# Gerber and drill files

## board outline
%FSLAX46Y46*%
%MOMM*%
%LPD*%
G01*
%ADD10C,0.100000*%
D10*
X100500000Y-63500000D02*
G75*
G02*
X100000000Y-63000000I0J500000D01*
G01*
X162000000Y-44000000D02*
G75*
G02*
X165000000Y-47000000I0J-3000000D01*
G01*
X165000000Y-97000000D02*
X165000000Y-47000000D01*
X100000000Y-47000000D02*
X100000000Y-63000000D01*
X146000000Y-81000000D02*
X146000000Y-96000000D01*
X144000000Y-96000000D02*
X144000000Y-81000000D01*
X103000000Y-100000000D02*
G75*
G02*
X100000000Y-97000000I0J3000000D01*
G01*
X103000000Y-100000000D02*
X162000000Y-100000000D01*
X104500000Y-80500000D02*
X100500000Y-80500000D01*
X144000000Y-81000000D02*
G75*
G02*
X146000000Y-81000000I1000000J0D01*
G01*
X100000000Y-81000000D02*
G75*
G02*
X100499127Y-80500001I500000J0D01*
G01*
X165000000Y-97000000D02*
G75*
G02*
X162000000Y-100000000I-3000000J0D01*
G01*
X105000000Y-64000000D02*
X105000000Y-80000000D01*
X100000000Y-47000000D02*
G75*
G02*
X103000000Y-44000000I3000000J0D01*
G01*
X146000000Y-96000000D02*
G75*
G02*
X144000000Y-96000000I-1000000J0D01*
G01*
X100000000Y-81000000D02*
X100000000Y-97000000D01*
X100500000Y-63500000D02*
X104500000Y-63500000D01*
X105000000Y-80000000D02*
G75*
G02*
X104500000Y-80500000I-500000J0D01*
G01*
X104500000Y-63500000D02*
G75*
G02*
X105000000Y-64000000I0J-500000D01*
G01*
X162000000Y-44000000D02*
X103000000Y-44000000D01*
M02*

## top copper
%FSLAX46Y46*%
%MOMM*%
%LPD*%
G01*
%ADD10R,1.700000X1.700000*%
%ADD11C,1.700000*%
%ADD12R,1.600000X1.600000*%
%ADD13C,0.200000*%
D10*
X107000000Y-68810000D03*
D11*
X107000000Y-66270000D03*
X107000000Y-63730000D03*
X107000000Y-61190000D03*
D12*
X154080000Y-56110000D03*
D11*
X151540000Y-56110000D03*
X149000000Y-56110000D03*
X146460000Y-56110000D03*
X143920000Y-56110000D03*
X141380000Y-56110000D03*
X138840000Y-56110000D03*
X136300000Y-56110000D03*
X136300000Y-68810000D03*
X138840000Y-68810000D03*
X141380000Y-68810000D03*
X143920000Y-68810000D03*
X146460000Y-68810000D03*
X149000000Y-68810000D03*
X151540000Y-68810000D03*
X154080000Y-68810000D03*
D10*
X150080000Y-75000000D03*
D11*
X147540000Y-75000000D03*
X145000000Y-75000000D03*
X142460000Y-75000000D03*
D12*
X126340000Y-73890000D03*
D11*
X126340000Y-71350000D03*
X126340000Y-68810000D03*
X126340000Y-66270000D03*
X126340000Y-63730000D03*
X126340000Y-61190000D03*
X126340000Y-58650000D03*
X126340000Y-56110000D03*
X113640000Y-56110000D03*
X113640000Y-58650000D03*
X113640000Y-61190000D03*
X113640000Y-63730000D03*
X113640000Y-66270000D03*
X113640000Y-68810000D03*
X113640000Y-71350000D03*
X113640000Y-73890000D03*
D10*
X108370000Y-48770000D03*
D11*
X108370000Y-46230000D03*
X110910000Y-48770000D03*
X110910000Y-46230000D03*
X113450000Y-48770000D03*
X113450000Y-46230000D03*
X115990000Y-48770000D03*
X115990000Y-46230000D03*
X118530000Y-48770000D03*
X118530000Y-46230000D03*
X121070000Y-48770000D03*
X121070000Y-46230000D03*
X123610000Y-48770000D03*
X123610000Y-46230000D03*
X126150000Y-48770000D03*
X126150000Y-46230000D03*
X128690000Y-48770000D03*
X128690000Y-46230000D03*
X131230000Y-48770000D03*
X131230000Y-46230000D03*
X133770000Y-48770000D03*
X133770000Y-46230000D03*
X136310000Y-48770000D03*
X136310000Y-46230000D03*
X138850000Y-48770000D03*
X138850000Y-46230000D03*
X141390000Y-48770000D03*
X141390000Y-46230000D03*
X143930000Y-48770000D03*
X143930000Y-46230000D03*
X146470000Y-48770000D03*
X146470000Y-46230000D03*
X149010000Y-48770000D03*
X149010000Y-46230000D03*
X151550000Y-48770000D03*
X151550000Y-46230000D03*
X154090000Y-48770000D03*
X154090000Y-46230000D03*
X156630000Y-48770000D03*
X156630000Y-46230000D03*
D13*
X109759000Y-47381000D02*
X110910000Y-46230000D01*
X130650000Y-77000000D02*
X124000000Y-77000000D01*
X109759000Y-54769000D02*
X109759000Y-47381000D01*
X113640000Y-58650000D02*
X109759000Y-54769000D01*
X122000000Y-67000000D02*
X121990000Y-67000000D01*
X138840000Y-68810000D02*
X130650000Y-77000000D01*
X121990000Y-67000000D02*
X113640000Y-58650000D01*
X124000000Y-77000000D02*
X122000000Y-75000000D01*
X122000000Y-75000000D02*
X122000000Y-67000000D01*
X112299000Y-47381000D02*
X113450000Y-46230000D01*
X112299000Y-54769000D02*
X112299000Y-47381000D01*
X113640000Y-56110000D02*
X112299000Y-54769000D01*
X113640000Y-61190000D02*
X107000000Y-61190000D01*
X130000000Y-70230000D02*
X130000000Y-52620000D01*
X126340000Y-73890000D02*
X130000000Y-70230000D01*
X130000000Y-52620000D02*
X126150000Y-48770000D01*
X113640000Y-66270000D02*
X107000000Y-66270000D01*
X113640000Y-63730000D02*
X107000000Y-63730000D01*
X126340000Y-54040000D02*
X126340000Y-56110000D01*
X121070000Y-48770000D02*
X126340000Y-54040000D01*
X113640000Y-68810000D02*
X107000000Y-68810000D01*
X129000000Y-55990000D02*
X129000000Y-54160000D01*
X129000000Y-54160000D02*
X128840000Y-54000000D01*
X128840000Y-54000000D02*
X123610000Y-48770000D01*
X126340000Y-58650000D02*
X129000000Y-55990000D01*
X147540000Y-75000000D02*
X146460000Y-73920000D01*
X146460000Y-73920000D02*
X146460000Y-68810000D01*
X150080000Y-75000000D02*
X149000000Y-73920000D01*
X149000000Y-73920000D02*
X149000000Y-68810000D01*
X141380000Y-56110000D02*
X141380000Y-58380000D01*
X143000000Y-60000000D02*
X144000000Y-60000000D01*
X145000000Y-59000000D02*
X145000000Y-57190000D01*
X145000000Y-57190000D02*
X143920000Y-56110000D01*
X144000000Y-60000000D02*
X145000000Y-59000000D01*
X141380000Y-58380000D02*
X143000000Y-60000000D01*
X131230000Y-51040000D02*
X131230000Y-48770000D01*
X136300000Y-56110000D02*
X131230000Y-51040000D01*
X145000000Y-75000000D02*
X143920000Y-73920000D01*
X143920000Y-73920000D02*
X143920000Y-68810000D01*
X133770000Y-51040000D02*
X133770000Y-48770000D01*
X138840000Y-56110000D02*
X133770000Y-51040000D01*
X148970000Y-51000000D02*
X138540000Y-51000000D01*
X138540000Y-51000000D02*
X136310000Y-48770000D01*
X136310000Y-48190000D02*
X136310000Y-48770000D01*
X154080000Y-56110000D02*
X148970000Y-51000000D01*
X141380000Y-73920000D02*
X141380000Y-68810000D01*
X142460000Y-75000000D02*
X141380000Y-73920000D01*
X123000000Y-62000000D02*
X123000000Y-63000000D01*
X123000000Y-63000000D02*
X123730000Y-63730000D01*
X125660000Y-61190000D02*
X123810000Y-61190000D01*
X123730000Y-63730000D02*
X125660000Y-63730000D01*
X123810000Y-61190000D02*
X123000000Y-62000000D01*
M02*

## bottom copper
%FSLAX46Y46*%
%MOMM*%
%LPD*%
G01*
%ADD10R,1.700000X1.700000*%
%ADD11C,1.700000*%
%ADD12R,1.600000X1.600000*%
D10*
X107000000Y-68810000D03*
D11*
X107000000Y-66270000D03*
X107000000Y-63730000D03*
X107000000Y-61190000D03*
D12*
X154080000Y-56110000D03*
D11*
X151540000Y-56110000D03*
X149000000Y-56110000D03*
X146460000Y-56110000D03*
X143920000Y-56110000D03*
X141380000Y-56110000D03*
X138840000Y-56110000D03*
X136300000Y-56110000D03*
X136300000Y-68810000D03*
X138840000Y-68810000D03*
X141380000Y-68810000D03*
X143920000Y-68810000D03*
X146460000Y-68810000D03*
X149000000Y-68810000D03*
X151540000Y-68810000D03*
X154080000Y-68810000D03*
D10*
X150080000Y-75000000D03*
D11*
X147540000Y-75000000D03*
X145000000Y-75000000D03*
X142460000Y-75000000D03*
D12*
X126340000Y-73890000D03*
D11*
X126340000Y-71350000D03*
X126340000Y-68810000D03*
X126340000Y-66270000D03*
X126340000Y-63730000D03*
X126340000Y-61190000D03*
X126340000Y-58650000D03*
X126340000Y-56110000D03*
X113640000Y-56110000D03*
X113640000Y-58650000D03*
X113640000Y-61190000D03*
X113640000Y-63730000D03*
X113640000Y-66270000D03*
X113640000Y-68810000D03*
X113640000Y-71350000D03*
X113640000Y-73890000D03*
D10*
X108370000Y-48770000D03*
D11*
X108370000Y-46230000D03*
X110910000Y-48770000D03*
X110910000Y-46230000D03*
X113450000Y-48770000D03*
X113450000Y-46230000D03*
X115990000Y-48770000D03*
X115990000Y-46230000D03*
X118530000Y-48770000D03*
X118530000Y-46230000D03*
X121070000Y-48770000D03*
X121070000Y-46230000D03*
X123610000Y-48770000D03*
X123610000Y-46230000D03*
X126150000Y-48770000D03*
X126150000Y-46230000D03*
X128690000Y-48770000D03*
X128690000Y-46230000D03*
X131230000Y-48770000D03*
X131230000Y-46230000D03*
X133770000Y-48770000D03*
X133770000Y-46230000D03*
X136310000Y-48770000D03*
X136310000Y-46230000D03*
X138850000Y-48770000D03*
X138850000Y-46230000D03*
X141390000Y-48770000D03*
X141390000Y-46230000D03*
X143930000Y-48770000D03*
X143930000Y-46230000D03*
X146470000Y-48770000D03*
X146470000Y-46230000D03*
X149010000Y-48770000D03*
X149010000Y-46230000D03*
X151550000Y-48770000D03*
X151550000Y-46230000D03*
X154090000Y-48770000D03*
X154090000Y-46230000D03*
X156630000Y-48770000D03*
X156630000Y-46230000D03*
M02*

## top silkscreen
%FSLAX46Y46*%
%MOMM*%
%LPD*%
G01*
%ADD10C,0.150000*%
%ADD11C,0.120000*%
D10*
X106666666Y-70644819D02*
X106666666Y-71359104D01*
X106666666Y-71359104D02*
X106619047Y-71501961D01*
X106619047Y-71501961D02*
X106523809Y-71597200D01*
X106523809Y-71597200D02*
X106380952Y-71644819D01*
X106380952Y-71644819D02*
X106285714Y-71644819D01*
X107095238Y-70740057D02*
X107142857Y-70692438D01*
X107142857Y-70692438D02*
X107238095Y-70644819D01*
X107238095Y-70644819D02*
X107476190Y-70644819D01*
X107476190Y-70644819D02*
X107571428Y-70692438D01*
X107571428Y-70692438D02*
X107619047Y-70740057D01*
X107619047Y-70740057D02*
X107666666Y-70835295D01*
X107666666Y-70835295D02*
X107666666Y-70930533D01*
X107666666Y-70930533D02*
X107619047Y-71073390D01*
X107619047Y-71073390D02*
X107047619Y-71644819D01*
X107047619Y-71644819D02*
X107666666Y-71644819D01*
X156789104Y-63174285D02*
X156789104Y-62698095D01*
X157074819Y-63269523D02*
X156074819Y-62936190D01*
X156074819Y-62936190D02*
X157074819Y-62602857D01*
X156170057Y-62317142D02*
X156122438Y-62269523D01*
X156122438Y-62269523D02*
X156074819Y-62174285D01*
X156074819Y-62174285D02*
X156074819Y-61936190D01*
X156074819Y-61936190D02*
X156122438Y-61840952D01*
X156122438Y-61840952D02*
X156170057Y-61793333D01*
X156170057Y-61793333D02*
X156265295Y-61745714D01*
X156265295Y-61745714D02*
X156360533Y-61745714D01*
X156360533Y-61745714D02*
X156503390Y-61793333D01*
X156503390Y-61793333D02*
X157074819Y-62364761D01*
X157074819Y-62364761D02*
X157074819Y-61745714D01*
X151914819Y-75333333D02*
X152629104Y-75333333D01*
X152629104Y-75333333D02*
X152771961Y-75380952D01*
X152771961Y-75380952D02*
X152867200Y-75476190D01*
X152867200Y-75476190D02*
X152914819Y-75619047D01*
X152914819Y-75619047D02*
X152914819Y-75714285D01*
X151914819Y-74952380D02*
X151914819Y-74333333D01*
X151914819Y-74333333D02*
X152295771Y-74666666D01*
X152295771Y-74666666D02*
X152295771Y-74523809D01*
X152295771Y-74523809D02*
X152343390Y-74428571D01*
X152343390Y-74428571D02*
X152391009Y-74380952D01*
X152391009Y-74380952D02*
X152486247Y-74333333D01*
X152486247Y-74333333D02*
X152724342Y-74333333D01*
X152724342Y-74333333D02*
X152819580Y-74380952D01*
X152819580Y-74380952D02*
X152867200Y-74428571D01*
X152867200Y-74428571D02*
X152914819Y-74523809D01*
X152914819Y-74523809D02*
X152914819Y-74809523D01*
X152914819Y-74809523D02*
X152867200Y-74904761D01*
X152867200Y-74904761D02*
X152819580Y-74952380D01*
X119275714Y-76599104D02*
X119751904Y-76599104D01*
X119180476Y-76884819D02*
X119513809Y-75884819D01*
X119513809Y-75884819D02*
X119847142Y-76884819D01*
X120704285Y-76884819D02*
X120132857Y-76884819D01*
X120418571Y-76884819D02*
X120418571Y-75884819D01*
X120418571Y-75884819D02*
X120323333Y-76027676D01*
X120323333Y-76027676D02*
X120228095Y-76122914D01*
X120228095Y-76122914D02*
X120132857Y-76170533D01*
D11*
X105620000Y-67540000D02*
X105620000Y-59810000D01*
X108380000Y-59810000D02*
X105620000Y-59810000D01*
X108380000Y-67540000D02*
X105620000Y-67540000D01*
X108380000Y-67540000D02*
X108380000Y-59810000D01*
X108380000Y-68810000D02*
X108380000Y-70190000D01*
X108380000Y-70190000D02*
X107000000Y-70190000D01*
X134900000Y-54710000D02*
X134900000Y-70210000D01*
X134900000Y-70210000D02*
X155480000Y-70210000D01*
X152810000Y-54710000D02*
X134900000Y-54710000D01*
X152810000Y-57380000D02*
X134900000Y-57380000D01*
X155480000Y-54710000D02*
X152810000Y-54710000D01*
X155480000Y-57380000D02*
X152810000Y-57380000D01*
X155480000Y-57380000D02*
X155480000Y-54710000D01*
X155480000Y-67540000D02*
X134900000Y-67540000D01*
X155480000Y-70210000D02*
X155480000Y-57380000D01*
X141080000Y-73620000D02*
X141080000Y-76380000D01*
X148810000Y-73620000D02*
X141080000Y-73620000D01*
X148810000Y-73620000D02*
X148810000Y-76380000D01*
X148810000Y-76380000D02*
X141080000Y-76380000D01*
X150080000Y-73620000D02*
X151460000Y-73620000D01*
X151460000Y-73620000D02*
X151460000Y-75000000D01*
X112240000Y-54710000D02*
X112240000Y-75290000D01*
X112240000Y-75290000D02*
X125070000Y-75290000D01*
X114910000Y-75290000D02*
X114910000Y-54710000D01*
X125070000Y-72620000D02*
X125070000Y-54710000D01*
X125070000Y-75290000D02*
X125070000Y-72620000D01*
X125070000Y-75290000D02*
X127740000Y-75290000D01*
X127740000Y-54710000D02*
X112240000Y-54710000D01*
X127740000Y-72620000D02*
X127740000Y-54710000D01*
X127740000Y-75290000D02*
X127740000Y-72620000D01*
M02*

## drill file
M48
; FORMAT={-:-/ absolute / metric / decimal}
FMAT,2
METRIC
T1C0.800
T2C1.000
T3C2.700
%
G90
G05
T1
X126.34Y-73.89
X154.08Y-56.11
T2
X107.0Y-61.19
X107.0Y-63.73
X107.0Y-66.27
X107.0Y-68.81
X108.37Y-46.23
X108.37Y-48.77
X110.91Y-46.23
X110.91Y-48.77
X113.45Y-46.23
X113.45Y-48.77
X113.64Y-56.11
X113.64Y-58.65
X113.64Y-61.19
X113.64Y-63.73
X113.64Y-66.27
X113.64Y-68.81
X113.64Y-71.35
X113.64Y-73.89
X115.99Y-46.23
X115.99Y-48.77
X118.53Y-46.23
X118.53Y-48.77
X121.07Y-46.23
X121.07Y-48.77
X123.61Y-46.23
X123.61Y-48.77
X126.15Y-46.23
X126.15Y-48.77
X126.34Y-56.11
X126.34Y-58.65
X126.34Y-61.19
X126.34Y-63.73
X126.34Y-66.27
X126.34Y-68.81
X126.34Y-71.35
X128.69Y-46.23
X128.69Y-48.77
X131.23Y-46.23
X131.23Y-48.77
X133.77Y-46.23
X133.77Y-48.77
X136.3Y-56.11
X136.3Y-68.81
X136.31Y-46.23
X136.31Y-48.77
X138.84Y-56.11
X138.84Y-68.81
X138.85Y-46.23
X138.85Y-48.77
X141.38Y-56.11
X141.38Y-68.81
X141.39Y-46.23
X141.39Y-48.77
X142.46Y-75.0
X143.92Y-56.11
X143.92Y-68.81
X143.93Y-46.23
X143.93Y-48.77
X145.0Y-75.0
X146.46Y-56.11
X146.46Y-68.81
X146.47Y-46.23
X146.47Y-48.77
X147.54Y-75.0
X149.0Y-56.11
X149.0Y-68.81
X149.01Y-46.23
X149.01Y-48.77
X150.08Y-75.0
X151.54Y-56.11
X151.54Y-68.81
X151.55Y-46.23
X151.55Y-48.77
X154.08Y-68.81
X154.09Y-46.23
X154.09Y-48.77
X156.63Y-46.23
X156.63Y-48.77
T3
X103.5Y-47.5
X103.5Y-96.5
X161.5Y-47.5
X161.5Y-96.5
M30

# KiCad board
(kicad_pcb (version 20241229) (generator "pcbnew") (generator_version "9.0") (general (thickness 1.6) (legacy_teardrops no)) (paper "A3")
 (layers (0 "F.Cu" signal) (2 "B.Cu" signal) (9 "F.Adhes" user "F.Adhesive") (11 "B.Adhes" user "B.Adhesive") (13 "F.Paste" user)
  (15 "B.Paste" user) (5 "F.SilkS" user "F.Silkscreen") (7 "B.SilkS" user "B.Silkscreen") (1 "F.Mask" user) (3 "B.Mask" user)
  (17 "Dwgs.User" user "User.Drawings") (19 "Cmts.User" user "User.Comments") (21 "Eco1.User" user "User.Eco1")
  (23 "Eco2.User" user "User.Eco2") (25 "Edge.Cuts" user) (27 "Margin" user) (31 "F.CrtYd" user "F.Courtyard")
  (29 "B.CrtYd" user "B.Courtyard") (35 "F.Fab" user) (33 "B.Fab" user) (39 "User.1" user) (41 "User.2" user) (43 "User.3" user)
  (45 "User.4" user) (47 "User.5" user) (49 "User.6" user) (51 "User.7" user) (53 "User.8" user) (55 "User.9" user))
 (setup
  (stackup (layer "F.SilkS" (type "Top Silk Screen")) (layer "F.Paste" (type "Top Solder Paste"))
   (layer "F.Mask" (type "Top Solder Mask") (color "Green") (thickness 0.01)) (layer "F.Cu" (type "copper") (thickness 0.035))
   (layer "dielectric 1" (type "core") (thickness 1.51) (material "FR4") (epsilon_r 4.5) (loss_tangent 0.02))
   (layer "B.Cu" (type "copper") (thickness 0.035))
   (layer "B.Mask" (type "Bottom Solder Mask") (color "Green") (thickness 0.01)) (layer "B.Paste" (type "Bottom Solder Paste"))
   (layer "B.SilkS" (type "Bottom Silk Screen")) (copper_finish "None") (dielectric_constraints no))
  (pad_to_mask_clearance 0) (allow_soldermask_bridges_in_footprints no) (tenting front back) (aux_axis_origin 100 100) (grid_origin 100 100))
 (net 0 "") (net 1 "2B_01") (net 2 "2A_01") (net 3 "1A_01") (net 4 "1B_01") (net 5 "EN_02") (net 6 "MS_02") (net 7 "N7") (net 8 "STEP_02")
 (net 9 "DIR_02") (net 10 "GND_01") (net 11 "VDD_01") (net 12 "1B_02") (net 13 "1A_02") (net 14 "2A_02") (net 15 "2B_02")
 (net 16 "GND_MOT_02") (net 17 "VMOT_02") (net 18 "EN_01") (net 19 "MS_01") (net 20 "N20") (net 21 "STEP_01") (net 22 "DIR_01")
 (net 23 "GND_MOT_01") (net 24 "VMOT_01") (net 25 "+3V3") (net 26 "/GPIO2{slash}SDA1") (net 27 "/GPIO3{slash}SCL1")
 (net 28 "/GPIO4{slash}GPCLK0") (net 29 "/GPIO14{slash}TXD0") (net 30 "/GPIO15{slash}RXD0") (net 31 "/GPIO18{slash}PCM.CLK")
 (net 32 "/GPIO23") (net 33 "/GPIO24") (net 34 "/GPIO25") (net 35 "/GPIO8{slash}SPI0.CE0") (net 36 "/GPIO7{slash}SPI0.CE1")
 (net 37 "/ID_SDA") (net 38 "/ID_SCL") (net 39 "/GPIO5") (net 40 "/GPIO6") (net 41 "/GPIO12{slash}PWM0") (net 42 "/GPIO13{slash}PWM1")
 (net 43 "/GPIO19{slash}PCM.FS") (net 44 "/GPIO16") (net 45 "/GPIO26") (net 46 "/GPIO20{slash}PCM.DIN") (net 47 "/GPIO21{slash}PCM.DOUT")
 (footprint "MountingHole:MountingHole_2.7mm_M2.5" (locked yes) (layer "F.Cu") (at 161.5 47.5)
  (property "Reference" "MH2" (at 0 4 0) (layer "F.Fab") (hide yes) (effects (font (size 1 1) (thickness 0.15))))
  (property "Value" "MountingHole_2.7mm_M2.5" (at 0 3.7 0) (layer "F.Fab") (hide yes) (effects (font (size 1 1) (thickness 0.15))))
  (pad "" np_thru_hole circle (at 0 0) (size 2.7 2.7) (drill 2.7) (layers "*.Cu" "*.Mask")))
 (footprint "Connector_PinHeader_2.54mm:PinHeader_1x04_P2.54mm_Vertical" (layer "F.Cu") (at 107 68.81 180)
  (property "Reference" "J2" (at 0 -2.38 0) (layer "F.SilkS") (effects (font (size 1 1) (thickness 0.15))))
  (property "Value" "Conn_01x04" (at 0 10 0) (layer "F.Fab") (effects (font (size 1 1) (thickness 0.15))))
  (fp_line (start 1.38 1.27) (end 1.38 9) (stroke (width 0.12) (type solid)) (layer "F.SilkS"))
  (fp_line (start -1.38 9) (end 1.38 9) (stroke (width 0.12) (type solid)) (layer "F.SilkS"))
  (fp_line (start -1.38 1.27) (end 1.38 1.27) (stroke (width 0.12) (type solid)) (layer "F.SilkS"))
  (fp_line (start -1.38 1.27) (end -1.38 9) (stroke (width 0.12) (type solid)) (layer "F.SilkS"))
  (fp_line (start -1.38 0) (end -1.38 -1.38) (stroke (width 0.12) (type solid)) (layer "F.SilkS"))
  (fp_line (start -1.38 -1.38) (end 0 -1.38) (stroke (width 0.12) (type solid)) (layer "F.SilkS"))
  (pad "1" thru_hole rect (at 0 0 180) (size 1.7 1.7) (drill 1) (layers "*.Cu" "*.Mask") (remove_unused_layers no) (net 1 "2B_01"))
  (pad "2" thru_hole circle (at 0 2.54 180) (size 1.7 1.7) (drill 1) (layers "*.Cu" "*.Mask") (remove_unused_layers no) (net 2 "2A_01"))
  (pad "3" thru_hole circle (at 0 5.08 180) (size 1.7 1.7) (drill 1) (layers "*.Cu" "*.Mask") (remove_unused_layers no) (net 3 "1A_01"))
  (pad "4" thru_hole circle (at 0 7.62 180) (size 1.7 1.7) (drill 1) (layers "*.Cu" "*.Mask") (remove_unused_layers no) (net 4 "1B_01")))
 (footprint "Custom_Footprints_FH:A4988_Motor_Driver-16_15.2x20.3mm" (layer "F.Cu") (at 154.08 56.11 -90)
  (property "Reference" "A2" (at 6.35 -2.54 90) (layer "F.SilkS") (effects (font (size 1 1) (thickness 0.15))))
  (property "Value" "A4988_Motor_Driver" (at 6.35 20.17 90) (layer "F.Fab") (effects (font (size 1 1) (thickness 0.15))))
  (fp_line (start -1.4 19.18) (end 14.1 19.18) (stroke (width 0.12) (type solid)) (layer "F.SilkS"))
  (fp_line (start 14.1 19.18) (end 14.1 -1.4) (stroke (width 0.12) (type solid)) (layer "F.SilkS"))
  (fp_line (start -1.4 1.27) (end -1.4 19.18) (stroke (width 0.12) (type solid)) (layer "F.SilkS"))
  (fp_line (start 1.27 1.27) (end 1.27 19.18) (stroke (width 0.12) (type solid)) (layer "F.SilkS"))
  (fp_line (start -1.4 -1.4) (end -1.4 1.27) (stroke (width 0.12) (type solid)) (layer "F.SilkS"))
  (fp_line (start 1.27 -1.4) (end 1.27 1.27) (stroke (width 0.12) (type solid)) (layer "F.SilkS"))
  (fp_line (start 1.27 -1.4) (end -1.4 -1.4) (stroke (width 0.12) (type solid)) (layer "F.SilkS"))
  (fp_line (start 11.43 -1.4) (end 11.43 19.18) (stroke (width 0.12) (type solid)) (layer "F.SilkS"))
  (fp_line (start 14.1 -1.4) (end 1.27 -1.4) (stroke (width 0.12) (type solid)) (layer "F.SilkS"))
  (pad "1" thru_hole rect (at 0 0 270) (size 1.6 1.6) (drill 0.8) (layers "*.Cu" "*.Mask") (remove_unused_layers no) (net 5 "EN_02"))
  (pad "2" thru_hole circle (at 0 2.54 270) (size 1.7 1.7) (drill 1) (layers "*.Cu" "*.Mask") (remove_unused_layers no) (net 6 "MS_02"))
  (pad "3" thru_hole circle (at 0 5.08 270) (size 1.7 1.7) (drill 1) (layers "*.Cu" "*.Mask") (remove_unused_layers no) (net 6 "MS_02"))
  (pad "4" thru_hole circle (at 0 7.62 270) (size 1.7 1.7) (drill 1) (layers "*.Cu" "*.Mask") (remove_unused_layers no) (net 6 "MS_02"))
  (pad "5" thru_hole circle (at 0 10.16 270) (size 1.7 1.7) (drill 1) (layers "*.Cu" "*.Mask") (remove_unused_layers no) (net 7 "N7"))
  (pad "6" thru_hole circle (at 0 12.7 270) (size 1.7 1.7) (drill 1) (layers "*.Cu" "*.Mask") (remove_unused_layers no) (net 7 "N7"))
  (pad "7" thru_hole circle (at 0 15.24 270) (size 1.7 1.7) (drill 1) (layers "*.Cu" "*.Mask") (remove_unused_layers no) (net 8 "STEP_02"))
  (pad "8" thru_hole circle (at 0 17.78 270) (size 1.7 1.7) (drill 1) (layers "*.Cu" "*.Mask") (remove_unused_layers no) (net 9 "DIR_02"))
  (pad "9" thru_hole circle (at 12.7 17.78 270) (size 1.7 1.7) (drill 1) (layers "*.Cu" "*.Mask") (remove_unused_layers no)
   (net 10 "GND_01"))
  (pad "10" thru_hole circle (at 12.7 15.24 270) (size 1.7 1.7) (drill 1) (layers "*.Cu" "*.Mask") (remove_unused_layers no)
   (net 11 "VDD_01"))
  (pad "11" thru_hole circle (at 12.7 12.7 270) (size 1.7 1.7) (drill 1) (layers "*.Cu" "*.Mask") (remove_unused_layers no) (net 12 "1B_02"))
  (pad "12" thru_hole circle (at 12.7 10.16 270) (size 1.7 1.7) (drill 1) (layers "*.Cu" "*.Mask") (remove_unused_layers no)
   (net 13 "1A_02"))
  (pad "13" thru_hole circle (at 12.7 7.62 270) (size 1.7 1.7) (drill 1) (layers "*.Cu" "*.Mask") (remove_unused_layers no) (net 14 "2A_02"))
  (pad "14" thru_hole circle (at 12.7 5.08 270) (size 1.7 1.7) (drill 1) (layers "*.Cu" "*.Mask") (remove_unused_layers no) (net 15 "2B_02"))
  (pad "15" thru_hole circle (at 12.7 2.54 270) (size 1.7 1.7) (drill 1) (layers "*.Cu" "*.Mask") (remove_unused_layers no)
   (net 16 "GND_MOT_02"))
  (pad "16" thru_hole circle (at 12.7 0 270) (size 1.7 1.7) (drill 1) (layers "*.Cu" "*.Mask") (remove_unused_layers no) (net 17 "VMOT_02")))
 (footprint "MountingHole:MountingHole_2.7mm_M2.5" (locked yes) (layer "F.Cu") (at 103.5 96.5)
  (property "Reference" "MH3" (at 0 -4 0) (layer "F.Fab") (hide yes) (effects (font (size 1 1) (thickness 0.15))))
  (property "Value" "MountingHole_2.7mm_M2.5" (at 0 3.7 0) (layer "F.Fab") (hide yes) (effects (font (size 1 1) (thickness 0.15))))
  (pad "" np_thru_hole circle (at 0 0) (size 2.7 2.7) (drill 2.7) (layers "*.Cu" "*.Mask")))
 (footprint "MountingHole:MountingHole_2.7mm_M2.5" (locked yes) (layer "F.Cu") (at 103.5 47.5)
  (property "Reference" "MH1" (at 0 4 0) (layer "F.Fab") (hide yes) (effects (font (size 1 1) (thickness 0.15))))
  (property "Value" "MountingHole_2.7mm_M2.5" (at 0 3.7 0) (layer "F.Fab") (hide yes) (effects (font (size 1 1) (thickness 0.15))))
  (pad "" np_thru_hole circle (at 0 0) (size 2.7 2.7) (drill 2.7) (layers "*.Cu" "*.Mask")))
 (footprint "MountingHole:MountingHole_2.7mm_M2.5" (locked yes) (layer "F.Cu") (at 161.5 96.5)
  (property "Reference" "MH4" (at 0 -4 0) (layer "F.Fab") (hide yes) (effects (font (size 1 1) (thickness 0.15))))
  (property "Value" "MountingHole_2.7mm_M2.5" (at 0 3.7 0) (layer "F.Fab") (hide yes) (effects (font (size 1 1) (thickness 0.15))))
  (pad "" np_thru_hole circle (at 0 0) (size 2.7 2.7) (drill 2.7) (layers "*.Cu" "*.Mask")))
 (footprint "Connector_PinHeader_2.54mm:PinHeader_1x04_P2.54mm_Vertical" (layer "F.Cu") (at 150.08 75 -90)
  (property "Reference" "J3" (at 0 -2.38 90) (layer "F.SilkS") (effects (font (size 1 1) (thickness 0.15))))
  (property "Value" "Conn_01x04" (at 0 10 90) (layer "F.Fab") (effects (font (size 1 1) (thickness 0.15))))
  (fp_line (start -1.38 9) (end 1.38 9) (stroke (width 0.12) (type solid)) (layer "F.SilkS"))
  (fp_line (start -1.38 1.27) (end -1.38 9) (stroke (width 0.12) (type solid)) (layer "F.SilkS"))
  (fp_line (start -1.38 1.27) (end 1.38 1.27) (stroke (width 0.12) (type solid)) (layer "F.SilkS"))
  (fp_line (start 1.38 1.27) (end 1.38 9) (stroke (width 0.12) (type solid)) (layer "F.SilkS"))
  (fp_line (start -1.38 0) (end -1.38 -1.38) (stroke (width 0.12) (type solid)) (layer "F.SilkS"))
  (fp_line (start -1.38 -1.38) (end 0 -1.38) (stroke (width 0.12) (type solid)) (layer "F.SilkS"))
  (pad "1" thru_hole rect (at 0 0 270) (size 1.7 1.7) (drill 1) (layers "*.Cu" "*.Mask") (remove_unused_layers no) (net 15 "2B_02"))
  (pad "2" thru_hole circle (at 0 2.54 270) (size 1.7 1.7) (drill 1) (layers "*.Cu" "*.Mask") (remove_unused_layers no) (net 14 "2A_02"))
  (pad "3" thru_hole circle (at 0 5.08 270) (size 1.7 1.7) (drill 1) (layers "*.Cu" "*.Mask") (remove_unused_layers no) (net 13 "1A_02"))
  (pad "4" thru_hole circle (at 0 7.62 270) (size 1.7 1.7) (drill 1) (layers "*.Cu" "*.Mask") (remove_unused_layers no) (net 12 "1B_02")))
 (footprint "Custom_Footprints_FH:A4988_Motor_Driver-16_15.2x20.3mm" (layer "F.Cu") (at 126.34 73.89 180)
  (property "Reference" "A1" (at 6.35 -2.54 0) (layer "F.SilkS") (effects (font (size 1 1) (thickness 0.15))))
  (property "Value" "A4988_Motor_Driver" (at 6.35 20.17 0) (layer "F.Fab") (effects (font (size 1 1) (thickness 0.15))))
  (fp_line (start 14.1 19.18) (end 14.1 -1.4) (stroke (width 0.12) (type solid)) (layer "F.SilkS"))
  (fp_line (start 14.1 -1.4) (end 1.27 -1.4) (stroke (width 0.12) (type solid)) (layer "F.SilkS"))
  (fp_line (start 11.43 -1.4) (end 11.43 19.18) (stroke (width 0.12) (type solid)) (layer "F.SilkS"))
  (fp_line (start 1.27 1.27) (end 1.27 19.18) (stroke (width 0.12) (type solid)) (layer "F.SilkS"))
  (fp_line (start 1.27 -1.4) (end 1.27 1.27) (stroke (width 0.12) (type solid)) (layer "F.SilkS"))
  (fp_line (start 1.27 -1.4) (end -1.4 -1.4) (stroke (width 0.12) (type solid)) (layer "F.SilkS"))
  (fp_line (start -1.4 19.18) (end 14.1 19.18) (stroke (width 0.12) (type solid)) (layer "F.SilkS"))
  (fp_line (start -1.4 1.27) (end -1.4 19.18) (stroke (width 0.12) (type solid)) (layer "F.SilkS"))
  (fp_line (start -1.4 -1.4) (end -1.4 1.27) (stroke (width 0.12) (type solid)) (layer "F.SilkS"))
  (pad "1" thru_hole rect (at 0 0 180) (size 1.6 1.6) (drill 0.8) (layers "*.Cu" "*.Mask") (remove_unused_layers no) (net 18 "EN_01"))
  (pad "2" thru_hole circle (at 0 2.54 180) (size 1.7 1.7) (drill 1) (layers "*.Cu" "*.Mask") (remove_unused_layers no) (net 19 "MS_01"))
  (pad "3" thru_hole circle (at 0 5.08 180) (size 1.7 1.7) (drill 1) (layers "*.Cu" "*.Mask") (remove_unused_layers no) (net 19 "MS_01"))
  (pad "4" thru_hole circle (at 0 7.62 180) (size 1.7 1.7) (drill 1) (layers "*.Cu" "*.Mask") (remove_unused_layers no) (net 19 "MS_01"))
  (pad "5" thru_hole circle (at 0 10.16 180) (size 1.7 1.7) (drill 1) (layers "*.Cu" "*.Mask") (remove_unused_layers no) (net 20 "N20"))
  (pad "6" thru_hole circle (at 0 12.7 180) (size 1.7 1.7) (drill 1) (layers "*.Cu" "*.Mask") (remove_unused_layers no) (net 20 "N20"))
  (pad "7" thru_hole circle (at 0 15.24 180) (size 1.7 1.7) (drill 1) (layers "*.Cu" "*.Mask") (remove_unused_layers no) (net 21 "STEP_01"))
  (pad "8" thru_hole circle (at 0 17.78 180) (size 1.7 1.7) (drill 1) (layers "*.Cu" "*.Mask") (remove_unused_layers no) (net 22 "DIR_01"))
  (pad "9" thru_hole circle (at 12.7 17.78 180) (size 1.7 1.7) (drill 1) (layers "*.Cu" "*.Mask") (remove_unused_layers no)
   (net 10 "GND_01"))
  (pad "10" thru_hole circle (at 12.7 15.24 180) (size 1.7 1.7) (drill 1) (layers "*.Cu" "*.Mask") (remove_unused_layers no)
   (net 11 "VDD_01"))
  (pad "11" thru_hole circle (at 12.7 12.7 180) (size 1.7 1.7) (drill 1) (layers "*.Cu" "*.Mask") (remove_unused_layers no) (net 4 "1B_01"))
  (pad "12" thru_hole circle (at 12.7 10.16 180) (size 1.7 1.7) (drill 1) (layers "*.Cu" "*.Mask") (remove_unused_layers no) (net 3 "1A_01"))
  (pad "13" thru_hole circle (at 12.7 7.62 180) (size 1.7 1.7) (drill 1) (layers "*.Cu" "*.Mask") (remove_unused_layers no) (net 2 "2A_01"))
  (pad "14" thru_hole circle (at 12.7 5.08 180) (size 1.7 1.7) (drill 1) (layers "*.Cu" "*.Mask") (remove_unused_layers no) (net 1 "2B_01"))
  (pad "15" thru_hole circle (at 12.7 2.54 180) (size 1.7 1.7) (drill 1) (layers "*.Cu" "*.Mask") (remove_unused_layers no)
   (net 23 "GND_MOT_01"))
  (pad "16" thru_hole circle (at 12.7 0 180) (size 1.7 1.7) (drill 1) (layers "*.Cu" "*.Mask") (remove_unused_layers no) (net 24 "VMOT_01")))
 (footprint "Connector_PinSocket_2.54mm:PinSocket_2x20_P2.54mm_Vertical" (layer "B.Cu") (at 108.37 48.77 -90)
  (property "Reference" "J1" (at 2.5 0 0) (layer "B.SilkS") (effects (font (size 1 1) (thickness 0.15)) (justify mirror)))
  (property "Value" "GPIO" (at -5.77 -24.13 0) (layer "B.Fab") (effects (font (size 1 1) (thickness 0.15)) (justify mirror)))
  (pad "1" thru_hole rect (at 0 0 270) (size 1.7 1.7) (drill 1) (layers "*.Cu" "*.Mask") (remove_unused_layers no) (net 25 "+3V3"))
  (pad "2" thru_hole circle (at -2.54 0 270) (size 1.7 1.7) (drill 1) (layers "*.Cu" "*.Mask") (remove_unused_layers no) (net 11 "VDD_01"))
  (pad "3" thru_hole circle (at 0 -2.54 270) (size 1.7 1.7) (drill 1) (layers "*.Cu" "*.Mask") (remove_unused_layers no)
   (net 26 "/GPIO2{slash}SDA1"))
  (pad "4" thru_hole circle (at -2.54 -2.54 270) (size 1.7 1.7) (drill 1) (layers "*.Cu" "*.Mask") (remove_unused_layers no)
   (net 11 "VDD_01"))
  (pad "5" thru_hole circle (at 0 -5.08 270) (size 1.7 1.7) (drill 1) (layers "*.Cu" "*.Mask") (remove_unused_layers no)
   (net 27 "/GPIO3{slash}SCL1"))
  (pad "6" thru_hole circle (at -2.54 -5.08 270) (size 1.7 1.7) (drill 1) (layers "*.Cu" "*.Mask") (remove_unused_layers no)
   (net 10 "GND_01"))
  (pad "7" thru_hole circle (at 0 -7.62 270) (size 1.7 1.7) (drill 1) (layers "*.Cu" "*.Mask") (remove_unused_layers no)
   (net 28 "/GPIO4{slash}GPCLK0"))
  (pad "8" thru_hole circle (at -2.54 -7.62 270) (size 1.7 1.7) (drill 1) (layers "*.Cu" "*.Mask") (remove_unused_layers no)
   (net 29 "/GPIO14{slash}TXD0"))
  (pad "9" thru_hole circle (at 0 -10.16 270) (size 1.7 1.7) (drill 1) (layers "*.Cu" "*.Mask") (remove_unused_layers no) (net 10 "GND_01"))
  (pad "10" thru_hole circle (at -2.54 -10.16 270) (size 1.7 1.7) (drill 1) (layers "*.Cu" "*.Mask") (remove_unused_layers no)
   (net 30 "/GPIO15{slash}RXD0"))
  (pad "11" thru_hole circle (at 0 -12.7 270) (size 1.7 1.7) (drill 1) (layers "*.Cu" "*.Mask") (remove_unused_layers no) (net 22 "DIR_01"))
  (pad "12" thru_hole circle (at -2.54 -12.7 270) (size 1.7 1.7) (drill 1) (layers "*.Cu" "*.Mask") (remove_unused_layers no)
   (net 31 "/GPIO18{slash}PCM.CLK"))
  (pad "13" thru_hole circle (at 0 -15.24 270) (size 1.7 1.7) (drill 1) (layers "*.Cu" "*.Mask") (remove_unused_layers no)
   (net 21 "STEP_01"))
  (pad "14" thru_hole circle (at -2.54 -15.24 270) (size 1.7 1.7) (drill 1) (layers "*.Cu" "*.Mask") (remove_unused_layers no)
   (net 10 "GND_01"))
  (pad "15" thru_hole circle (at 0 -17.78 270) (size 1.7 1.7) (drill 1) (layers "*.Cu" "*.Mask") (remove_unused_layers no) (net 18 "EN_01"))
  (pad "16" thru_hole circle (at -2.54 -17.78 270) (size 1.7 1.7) (drill 1) (layers "*.Cu" "*.Mask") (remove_unused_layers no)
   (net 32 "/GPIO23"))
  (pad "17" thru_hole circle (at 0 -20.32 270) (size 1.7 1.7) (drill 1) (layers "*.Cu" "*.Mask") (remove_unused_layers no) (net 25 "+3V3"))
  (pad "18" thru_hole circle (at -2.54 -20.32 270) (size 1.7 1.7) (drill 1) (layers "*.Cu" "*.Mask") (remove_unused_layers no)
   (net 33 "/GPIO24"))
  (pad "19" thru_hole circle (at 0 -22.86 270) (size 1.7 1.7) (drill 1) (layers "*.Cu" "*.Mask") (remove_unused_layers no) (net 9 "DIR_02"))
  (pad "20" thru_hole circle (at -2.54 -22.86 270) (size 1.7 1.7) (drill 1) (layers "*.Cu" "*.Mask") (remove_unused_layers no)
   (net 10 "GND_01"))
  (pad "21" thru_hole circle (at 0 -25.4 270) (size 1.7 1.7) (drill 1) (layers "*.Cu" "*.Mask") (remove_unused_layers no) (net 8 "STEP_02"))
  (pad "22" thru_hole circle (at -2.54 -25.4 270) (size 1.7 1.7) (drill 1) (layers "*.Cu" "*.Mask") (remove_unused_layers no)
   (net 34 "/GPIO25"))
  (pad "23" thru_hole circle (at 0 -27.94 270) (size 1.7 1.7) (drill 1) (layers "*.Cu" "*.Mask") (remove_unused_layers no) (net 5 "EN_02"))
  (pad "24" thru_hole circle (at -2.54 -27.94 270) (size 1.7 1.7) (drill 1) (layers "*.Cu" "*.Mask") (remove_unused_layers no)
   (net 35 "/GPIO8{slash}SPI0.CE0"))
  (pad "25" thru_hole circle (at 0 -30.48 270) (size 1.7 1.7) (drill 1) (layers "*.Cu" "*.Mask") (remove_unused_layers no) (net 10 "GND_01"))
  (pad "26" thru_hole circle (at -2.54 -30.48 270) (size 1.7 1.7) (drill 1) (layers "*.Cu" "*.Mask") (remove_unused_layers no)
   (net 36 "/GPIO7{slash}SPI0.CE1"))
  (pad "27" thru_hole circle (at 0 -33.02 270) (size 1.7 1.7) (drill 1) (layers "*.Cu" "*.Mask") (remove_unused_layers no)
   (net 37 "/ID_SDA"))
  (pad "28" thru_hole circle (at -2.54 -33.02 270) (size 1.7 1.7) (drill 1) (layers "*.Cu" "*.Mask") (remove_unused_layers no)
   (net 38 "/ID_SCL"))
  (pad "29" thru_hole circle (at 0 -35.56 270) (size 1.7 1.7) (drill 1) (layers "*.Cu" "*.Mask") (remove_unused_layers no) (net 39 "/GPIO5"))
  (pad "30" thru_hole circle (at -2.54 -35.56 270) (size 1.7 1.7) (drill 1) (layers "*.Cu" "*.Mask") (remove_unused_layers no)
   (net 10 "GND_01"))
  (pad "31" thru_hole circle (at 0 -38.1 270) (size 1.7 1.7) (drill 1) (layers "*.Cu" "*.Mask") (remove_unused_layers no) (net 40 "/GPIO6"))
  (pad "32" thru_hole circle (at -2.54 -38.1 270) (size 1.7 1.7) (drill 1) (layers "*.Cu" "*.Mask") (remove_unused_layers no)
   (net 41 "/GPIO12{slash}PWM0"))
  (pad "33" thru_hole circle (at 0 -40.64 270) (size 1.7 1.7) (drill 1) (layers "*.Cu" "*.Mask") (remove_unused_layers no)
   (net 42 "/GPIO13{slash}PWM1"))
  (pad "34" thru_hole circle (at -2.54 -40.64 270) (size 1.7 1.7) (drill 1) (layers "*.Cu" "*.Mask") (remove_unused_layers no)
   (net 10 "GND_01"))
  (pad "35" thru_hole circle (at 0 -43.18 270) (size 1.7 1.7) (drill 1) (layers "*.Cu" "*.Mask") (remove_unused_layers no)
   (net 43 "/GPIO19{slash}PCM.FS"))
  (pad "36" thru_hole circle (at -2.54 -43.18 270) (size 1.7 1.7) (drill 1) (layers "*.Cu" "*.Mask") (remove_unused_layers no)
   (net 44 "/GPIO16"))
  (pad "37" thru_hole circle (at 0 -45.72 270) (size 1.7 1.7) (drill 1) (layers "*.Cu" "*.Mask") (remove_unused_layers no)
   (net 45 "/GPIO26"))
  (pad "38" thru_hole circle (at -2.54 -45.72 270) (size 1.7 1.7) (drill 1) (layers "*.Cu" "*.Mask") (remove_unused_layers no)
   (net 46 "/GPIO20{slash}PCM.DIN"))
  (pad "39" thru_hole circle (at 0 -48.26 270) (size 1.7 1.7) (drill 1) (layers "*.Cu" "*.Mask") (remove_unused_layers no) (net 10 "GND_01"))
  (pad "40" thru_hole circle (at -2.54 -48.26 270) (size 1.7 1.7) (drill 1) (layers "*.Cu" "*.Mask") (remove_unused_layers no)
   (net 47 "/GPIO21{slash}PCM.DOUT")))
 (gr_arc (start 100.5 63.5) (mid 100.146447 63.353553) (end 100 63) (stroke (width 0.1) (type solid)) (layer "Edge.Cuts"))
 (gr_arc (start 162 44) (mid 164.12132 44.87868) (end 165 47) (stroke (width 0.1) (type solid)) (layer "Edge.Cuts"))
 (gr_line (start 165 97) (end 165 47) (stroke (width 0.1) (type solid)) (layer "Edge.Cuts"))
 (gr_line (start 100 47) (end 100 63) (stroke (width 0.1) (type solid)) (layer "Edge.Cuts"))
 (gr_line (start 146 81) (end 146 96) (stroke (width 0.1) (type solid)) (layer "Edge.Cuts"))
 (gr_line (start 144 96) (end 144 81) (stroke (width 0.1) (type solid)) (layer "Edge.Cuts"))
 (gr_arc (start 103 100) (mid 100.87868 99.12132) (end 100 97) (stroke (width 0.1) (type solid)) (layer "Edge.Cuts"))
 (gr_line (start 103 100) (end 162 100) (stroke (width 0.1) (type solid)) (layer "Edge.Cuts"))
 (gr_line (start 104.5 80.5) (end 100.5 80.5) (stroke (width 0.1) (type solid)) (layer "Edge.Cuts"))
 (gr_arc (start 144 81) (mid 145 80) (end 146 81) (stroke (width 0.1) (type solid)) (layer "Edge.Cuts"))
 (gr_arc (start 100 81) (mid 100.146138 80.646755) (end 100.499127 80.500001) (stroke (width 0.1) (type solid)) (layer "Edge.Cuts"))
 (gr_arc (start 165 97) (mid 164.12132 99.12132) (end 162 100) (stroke (width 0.1) (type solid)) (layer "Edge.Cuts"))
 (gr_line (start 105 64) (end 105 80) (stroke (width 0.1) (type solid)) (layer "Edge.Cuts"))
 (gr_arc (start 100 47) (mid 100.87868 44.87868) (end 103 44) (stroke (width 0.1) (type solid)) (layer "Edge.Cuts"))
 (gr_arc (start 146 96) (mid 145 97) (end 144 96) (stroke (width 0.1) (type solid)) (layer "Edge.Cuts"))
 (gr_line (start 100 81) (end 100 97) (stroke (width 0.1) (type solid)) (layer "Edge.Cuts"))
 (gr_line (start 100.5 63.5) (end 104.5 63.5) (stroke (width 0.1) (type solid)) (layer "Edge.Cuts"))
 (gr_arc (start 105 80) (mid 104.853553 80.353553) (end 104.5 80.5) (stroke (width 0.1) (type solid)) (layer "Edge.Cuts"))
 (gr_arc (start 104.5 63.5) (mid 104.853553 63.646447) (end 105 64) (stroke (width 0.1) (type solid)) (layer "Edge.Cuts"))
 (gr_line (start 162 44) (end 103 44) (stroke (width 0.1) (type solid)) (layer "Edge.Cuts"))
 (segment (start 109.759 47.381) (end 110.91 46.23) (width 0.2) (layer "F.Cu") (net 11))
 (segment (start 130.65 77) (end 124 77) (width 0.2) (layer "F.Cu") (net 11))
 (segment (start 109.759 54.769) (end 109.759 47.381) (width 0.2) (layer "F.Cu") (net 11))
 (segment (start 113.64 58.65) (end 109.759 54.769) (width 0.2) (layer "F.Cu") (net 11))
 (segment (start 122 67) (end 121.99 67) (width 0.2) (layer "F.Cu") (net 11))
 (segment (start 138.84 68.81) (end 130.65 77) (width 0.2) (layer "F.Cu") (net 11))
 (segment (start 121.99 67) (end 113.64 58.65) (width 0.2) (layer "F.Cu") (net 11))
 (segment (start 124 77) (end 122 75) (width 0.2) (layer "F.Cu") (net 11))
 (segment (start 122 75) (end 122 67) (width 0.2) (layer "F.Cu") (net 11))
 (segment (start 112.299 47.381) (end 113.45 46.23) (width 0.2) (layer "F.Cu") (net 10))
 (segment (start 112.299 54.769) (end 112.299 47.381) (width 0.2) (layer "F.Cu") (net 10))
 (segment (start 113.64 56.11) (end 112.299 54.769) (width 0.2) (layer "F.Cu") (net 10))
 (segment (start 113.64 61.19) (end 107 61.19) (width 0.2) (layer "F.Cu") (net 4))
 (segment (start 130 70.23) (end 130 52.62) (width 0.2) (layer "F.Cu") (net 18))
 (segment (start 126.34 73.89) (end 130 70.23) (width 0.2) (layer "F.Cu") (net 18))
 (segment (start 130 52.62) (end 126.15 48.77) (width 0.2) (layer "F.Cu") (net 18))
 (segment (start 113.64 66.27) (end 107 66.27) (width 0.2) (layer "F.Cu") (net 2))
 (segment (start 113.64 63.73) (end 107 63.73) (width 0.2) (layer "F.Cu") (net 3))
 (segment (start 126.34 54.04) (end 126.34 56.11) (width 0.2) (layer "F.Cu") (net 22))
 (segment (start 121.07 48.77) (end 126.34 54.04) (width 0.2) (layer "F.Cu") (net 22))
 (segment (start 113.64 68.81) (end 107 68.81) (width 0.2) (layer "F.Cu") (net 1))
 (segment (start 129 55.99) (end 129 54.16) (width 0.2) (layer "F.Cu") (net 21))
 (segment (start 129 54.16) (end 128.84 54) (width 0.2) (layer "F.Cu") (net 21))
 (segment (start 128.84 54) (end 123.61 48.77) (width 0.2) (layer "F.Cu") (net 21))
 (segment (start 126.34 58.65) (end 129 55.99) (width 0.2) (layer "F.Cu") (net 21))
 (segment (start 147.54 75) (end 146.46 73.92) (width 0.2) (layer "F.Cu") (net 14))
 (segment (start 146.46 73.92) (end 146.46 68.81) (width 0.2) (layer "F.Cu") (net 14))
 (segment (start 150.08 75) (end 149 73.92) (width 0.2) (layer "F.Cu") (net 15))
 (segment (start 149 73.92) (end 149 68.81) (width 0.2) (layer "F.Cu") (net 15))
 (segment (start 141.38 56.11) (end 141.38 58.38) (width 0.2) (layer "F.Cu") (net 7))
 (segment (start 143 60) (end 144 60) (width 0.2) (layer "F.Cu") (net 7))
 (segment (start 145 59) (end 145 57.19) (width 0.2) (layer "F.Cu") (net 7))
 (segment (start 145 57.19) (end 143.92 56.11) (width 0.2) (layer "F.Cu") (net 7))
 (segment (start 144 60) (end 145 59) (width 0.2) (layer "F.Cu") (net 7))
 (segment (start 141.38 58.38) (end 143 60) (width 0.2) (layer "F.Cu") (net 7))
 (segment (start 131.23 51.04) (end 131.23 48.77) (width 0.2) (layer "F.Cu") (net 9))
 (segment (start 136.3 56.11) (end 131.23 51.04) (width 0.2) (layer "F.Cu") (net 9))
 (segment (start 145 75) (end 143.92 73.92) (width 0.2) (layer "F.Cu") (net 13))
 (segment (start 143.92 73.92) (end 143.92 68.81) (width 0.2) (layer "F.Cu") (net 13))
 (segment (start 133.77 51.04) (end 133.77 48.77) (width 0.2) (layer "F.Cu") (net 8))
 (segment (start 138.84 56.11) (end 133.77 51.04) (width 0.2) (layer "F.Cu") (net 8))
 (segment (start 148.97 51) (end 138.54 51) (width 0.2) (layer "F.Cu") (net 5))
 (segment (start 138.54 51) (end 136.31 48.77) (width 0.2) (layer "F.Cu") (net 5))
 (segment (start 136.31 48.19) (end 136.31 48.77) (width 0.2) (layer "F.Cu") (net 5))
 (segment (start 154.08 56.11) (end 148.97 51) (width 0.2) (layer "F.Cu") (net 5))
 (segment (start 141.38 73.92) (end 141.38 68.81) (width 0.2) (layer "F.Cu") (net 12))
 (segment (start 142.46 75) (end 141.38 73.92) (width 0.2) (layer "F.Cu") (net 12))
 (segment (start 123 62) (end 123 63) (width 0.2) (layer "F.Cu") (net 20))
 (segment (start 123 63) (end 123.73 63.73) (width 0.2) (layer "F.Cu") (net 20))
 (segment (start 125.66 61.19) (end 123.81 61.19) (width 0.2) (layer "F.Cu") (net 20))
 (segment (start 123.73 63.73) (end 125.66 63.73) (width 0.2) (layer "F.Cu") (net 20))
 (segment (start 123.81 61.19) (end 123 62) (width 0.2) (layer "F.Cu") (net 20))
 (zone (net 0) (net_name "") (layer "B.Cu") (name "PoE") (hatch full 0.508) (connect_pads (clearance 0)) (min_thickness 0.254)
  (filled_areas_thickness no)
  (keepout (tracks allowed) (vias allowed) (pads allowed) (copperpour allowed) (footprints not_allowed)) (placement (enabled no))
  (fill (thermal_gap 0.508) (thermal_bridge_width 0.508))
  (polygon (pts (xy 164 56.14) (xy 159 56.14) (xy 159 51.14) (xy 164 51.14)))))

